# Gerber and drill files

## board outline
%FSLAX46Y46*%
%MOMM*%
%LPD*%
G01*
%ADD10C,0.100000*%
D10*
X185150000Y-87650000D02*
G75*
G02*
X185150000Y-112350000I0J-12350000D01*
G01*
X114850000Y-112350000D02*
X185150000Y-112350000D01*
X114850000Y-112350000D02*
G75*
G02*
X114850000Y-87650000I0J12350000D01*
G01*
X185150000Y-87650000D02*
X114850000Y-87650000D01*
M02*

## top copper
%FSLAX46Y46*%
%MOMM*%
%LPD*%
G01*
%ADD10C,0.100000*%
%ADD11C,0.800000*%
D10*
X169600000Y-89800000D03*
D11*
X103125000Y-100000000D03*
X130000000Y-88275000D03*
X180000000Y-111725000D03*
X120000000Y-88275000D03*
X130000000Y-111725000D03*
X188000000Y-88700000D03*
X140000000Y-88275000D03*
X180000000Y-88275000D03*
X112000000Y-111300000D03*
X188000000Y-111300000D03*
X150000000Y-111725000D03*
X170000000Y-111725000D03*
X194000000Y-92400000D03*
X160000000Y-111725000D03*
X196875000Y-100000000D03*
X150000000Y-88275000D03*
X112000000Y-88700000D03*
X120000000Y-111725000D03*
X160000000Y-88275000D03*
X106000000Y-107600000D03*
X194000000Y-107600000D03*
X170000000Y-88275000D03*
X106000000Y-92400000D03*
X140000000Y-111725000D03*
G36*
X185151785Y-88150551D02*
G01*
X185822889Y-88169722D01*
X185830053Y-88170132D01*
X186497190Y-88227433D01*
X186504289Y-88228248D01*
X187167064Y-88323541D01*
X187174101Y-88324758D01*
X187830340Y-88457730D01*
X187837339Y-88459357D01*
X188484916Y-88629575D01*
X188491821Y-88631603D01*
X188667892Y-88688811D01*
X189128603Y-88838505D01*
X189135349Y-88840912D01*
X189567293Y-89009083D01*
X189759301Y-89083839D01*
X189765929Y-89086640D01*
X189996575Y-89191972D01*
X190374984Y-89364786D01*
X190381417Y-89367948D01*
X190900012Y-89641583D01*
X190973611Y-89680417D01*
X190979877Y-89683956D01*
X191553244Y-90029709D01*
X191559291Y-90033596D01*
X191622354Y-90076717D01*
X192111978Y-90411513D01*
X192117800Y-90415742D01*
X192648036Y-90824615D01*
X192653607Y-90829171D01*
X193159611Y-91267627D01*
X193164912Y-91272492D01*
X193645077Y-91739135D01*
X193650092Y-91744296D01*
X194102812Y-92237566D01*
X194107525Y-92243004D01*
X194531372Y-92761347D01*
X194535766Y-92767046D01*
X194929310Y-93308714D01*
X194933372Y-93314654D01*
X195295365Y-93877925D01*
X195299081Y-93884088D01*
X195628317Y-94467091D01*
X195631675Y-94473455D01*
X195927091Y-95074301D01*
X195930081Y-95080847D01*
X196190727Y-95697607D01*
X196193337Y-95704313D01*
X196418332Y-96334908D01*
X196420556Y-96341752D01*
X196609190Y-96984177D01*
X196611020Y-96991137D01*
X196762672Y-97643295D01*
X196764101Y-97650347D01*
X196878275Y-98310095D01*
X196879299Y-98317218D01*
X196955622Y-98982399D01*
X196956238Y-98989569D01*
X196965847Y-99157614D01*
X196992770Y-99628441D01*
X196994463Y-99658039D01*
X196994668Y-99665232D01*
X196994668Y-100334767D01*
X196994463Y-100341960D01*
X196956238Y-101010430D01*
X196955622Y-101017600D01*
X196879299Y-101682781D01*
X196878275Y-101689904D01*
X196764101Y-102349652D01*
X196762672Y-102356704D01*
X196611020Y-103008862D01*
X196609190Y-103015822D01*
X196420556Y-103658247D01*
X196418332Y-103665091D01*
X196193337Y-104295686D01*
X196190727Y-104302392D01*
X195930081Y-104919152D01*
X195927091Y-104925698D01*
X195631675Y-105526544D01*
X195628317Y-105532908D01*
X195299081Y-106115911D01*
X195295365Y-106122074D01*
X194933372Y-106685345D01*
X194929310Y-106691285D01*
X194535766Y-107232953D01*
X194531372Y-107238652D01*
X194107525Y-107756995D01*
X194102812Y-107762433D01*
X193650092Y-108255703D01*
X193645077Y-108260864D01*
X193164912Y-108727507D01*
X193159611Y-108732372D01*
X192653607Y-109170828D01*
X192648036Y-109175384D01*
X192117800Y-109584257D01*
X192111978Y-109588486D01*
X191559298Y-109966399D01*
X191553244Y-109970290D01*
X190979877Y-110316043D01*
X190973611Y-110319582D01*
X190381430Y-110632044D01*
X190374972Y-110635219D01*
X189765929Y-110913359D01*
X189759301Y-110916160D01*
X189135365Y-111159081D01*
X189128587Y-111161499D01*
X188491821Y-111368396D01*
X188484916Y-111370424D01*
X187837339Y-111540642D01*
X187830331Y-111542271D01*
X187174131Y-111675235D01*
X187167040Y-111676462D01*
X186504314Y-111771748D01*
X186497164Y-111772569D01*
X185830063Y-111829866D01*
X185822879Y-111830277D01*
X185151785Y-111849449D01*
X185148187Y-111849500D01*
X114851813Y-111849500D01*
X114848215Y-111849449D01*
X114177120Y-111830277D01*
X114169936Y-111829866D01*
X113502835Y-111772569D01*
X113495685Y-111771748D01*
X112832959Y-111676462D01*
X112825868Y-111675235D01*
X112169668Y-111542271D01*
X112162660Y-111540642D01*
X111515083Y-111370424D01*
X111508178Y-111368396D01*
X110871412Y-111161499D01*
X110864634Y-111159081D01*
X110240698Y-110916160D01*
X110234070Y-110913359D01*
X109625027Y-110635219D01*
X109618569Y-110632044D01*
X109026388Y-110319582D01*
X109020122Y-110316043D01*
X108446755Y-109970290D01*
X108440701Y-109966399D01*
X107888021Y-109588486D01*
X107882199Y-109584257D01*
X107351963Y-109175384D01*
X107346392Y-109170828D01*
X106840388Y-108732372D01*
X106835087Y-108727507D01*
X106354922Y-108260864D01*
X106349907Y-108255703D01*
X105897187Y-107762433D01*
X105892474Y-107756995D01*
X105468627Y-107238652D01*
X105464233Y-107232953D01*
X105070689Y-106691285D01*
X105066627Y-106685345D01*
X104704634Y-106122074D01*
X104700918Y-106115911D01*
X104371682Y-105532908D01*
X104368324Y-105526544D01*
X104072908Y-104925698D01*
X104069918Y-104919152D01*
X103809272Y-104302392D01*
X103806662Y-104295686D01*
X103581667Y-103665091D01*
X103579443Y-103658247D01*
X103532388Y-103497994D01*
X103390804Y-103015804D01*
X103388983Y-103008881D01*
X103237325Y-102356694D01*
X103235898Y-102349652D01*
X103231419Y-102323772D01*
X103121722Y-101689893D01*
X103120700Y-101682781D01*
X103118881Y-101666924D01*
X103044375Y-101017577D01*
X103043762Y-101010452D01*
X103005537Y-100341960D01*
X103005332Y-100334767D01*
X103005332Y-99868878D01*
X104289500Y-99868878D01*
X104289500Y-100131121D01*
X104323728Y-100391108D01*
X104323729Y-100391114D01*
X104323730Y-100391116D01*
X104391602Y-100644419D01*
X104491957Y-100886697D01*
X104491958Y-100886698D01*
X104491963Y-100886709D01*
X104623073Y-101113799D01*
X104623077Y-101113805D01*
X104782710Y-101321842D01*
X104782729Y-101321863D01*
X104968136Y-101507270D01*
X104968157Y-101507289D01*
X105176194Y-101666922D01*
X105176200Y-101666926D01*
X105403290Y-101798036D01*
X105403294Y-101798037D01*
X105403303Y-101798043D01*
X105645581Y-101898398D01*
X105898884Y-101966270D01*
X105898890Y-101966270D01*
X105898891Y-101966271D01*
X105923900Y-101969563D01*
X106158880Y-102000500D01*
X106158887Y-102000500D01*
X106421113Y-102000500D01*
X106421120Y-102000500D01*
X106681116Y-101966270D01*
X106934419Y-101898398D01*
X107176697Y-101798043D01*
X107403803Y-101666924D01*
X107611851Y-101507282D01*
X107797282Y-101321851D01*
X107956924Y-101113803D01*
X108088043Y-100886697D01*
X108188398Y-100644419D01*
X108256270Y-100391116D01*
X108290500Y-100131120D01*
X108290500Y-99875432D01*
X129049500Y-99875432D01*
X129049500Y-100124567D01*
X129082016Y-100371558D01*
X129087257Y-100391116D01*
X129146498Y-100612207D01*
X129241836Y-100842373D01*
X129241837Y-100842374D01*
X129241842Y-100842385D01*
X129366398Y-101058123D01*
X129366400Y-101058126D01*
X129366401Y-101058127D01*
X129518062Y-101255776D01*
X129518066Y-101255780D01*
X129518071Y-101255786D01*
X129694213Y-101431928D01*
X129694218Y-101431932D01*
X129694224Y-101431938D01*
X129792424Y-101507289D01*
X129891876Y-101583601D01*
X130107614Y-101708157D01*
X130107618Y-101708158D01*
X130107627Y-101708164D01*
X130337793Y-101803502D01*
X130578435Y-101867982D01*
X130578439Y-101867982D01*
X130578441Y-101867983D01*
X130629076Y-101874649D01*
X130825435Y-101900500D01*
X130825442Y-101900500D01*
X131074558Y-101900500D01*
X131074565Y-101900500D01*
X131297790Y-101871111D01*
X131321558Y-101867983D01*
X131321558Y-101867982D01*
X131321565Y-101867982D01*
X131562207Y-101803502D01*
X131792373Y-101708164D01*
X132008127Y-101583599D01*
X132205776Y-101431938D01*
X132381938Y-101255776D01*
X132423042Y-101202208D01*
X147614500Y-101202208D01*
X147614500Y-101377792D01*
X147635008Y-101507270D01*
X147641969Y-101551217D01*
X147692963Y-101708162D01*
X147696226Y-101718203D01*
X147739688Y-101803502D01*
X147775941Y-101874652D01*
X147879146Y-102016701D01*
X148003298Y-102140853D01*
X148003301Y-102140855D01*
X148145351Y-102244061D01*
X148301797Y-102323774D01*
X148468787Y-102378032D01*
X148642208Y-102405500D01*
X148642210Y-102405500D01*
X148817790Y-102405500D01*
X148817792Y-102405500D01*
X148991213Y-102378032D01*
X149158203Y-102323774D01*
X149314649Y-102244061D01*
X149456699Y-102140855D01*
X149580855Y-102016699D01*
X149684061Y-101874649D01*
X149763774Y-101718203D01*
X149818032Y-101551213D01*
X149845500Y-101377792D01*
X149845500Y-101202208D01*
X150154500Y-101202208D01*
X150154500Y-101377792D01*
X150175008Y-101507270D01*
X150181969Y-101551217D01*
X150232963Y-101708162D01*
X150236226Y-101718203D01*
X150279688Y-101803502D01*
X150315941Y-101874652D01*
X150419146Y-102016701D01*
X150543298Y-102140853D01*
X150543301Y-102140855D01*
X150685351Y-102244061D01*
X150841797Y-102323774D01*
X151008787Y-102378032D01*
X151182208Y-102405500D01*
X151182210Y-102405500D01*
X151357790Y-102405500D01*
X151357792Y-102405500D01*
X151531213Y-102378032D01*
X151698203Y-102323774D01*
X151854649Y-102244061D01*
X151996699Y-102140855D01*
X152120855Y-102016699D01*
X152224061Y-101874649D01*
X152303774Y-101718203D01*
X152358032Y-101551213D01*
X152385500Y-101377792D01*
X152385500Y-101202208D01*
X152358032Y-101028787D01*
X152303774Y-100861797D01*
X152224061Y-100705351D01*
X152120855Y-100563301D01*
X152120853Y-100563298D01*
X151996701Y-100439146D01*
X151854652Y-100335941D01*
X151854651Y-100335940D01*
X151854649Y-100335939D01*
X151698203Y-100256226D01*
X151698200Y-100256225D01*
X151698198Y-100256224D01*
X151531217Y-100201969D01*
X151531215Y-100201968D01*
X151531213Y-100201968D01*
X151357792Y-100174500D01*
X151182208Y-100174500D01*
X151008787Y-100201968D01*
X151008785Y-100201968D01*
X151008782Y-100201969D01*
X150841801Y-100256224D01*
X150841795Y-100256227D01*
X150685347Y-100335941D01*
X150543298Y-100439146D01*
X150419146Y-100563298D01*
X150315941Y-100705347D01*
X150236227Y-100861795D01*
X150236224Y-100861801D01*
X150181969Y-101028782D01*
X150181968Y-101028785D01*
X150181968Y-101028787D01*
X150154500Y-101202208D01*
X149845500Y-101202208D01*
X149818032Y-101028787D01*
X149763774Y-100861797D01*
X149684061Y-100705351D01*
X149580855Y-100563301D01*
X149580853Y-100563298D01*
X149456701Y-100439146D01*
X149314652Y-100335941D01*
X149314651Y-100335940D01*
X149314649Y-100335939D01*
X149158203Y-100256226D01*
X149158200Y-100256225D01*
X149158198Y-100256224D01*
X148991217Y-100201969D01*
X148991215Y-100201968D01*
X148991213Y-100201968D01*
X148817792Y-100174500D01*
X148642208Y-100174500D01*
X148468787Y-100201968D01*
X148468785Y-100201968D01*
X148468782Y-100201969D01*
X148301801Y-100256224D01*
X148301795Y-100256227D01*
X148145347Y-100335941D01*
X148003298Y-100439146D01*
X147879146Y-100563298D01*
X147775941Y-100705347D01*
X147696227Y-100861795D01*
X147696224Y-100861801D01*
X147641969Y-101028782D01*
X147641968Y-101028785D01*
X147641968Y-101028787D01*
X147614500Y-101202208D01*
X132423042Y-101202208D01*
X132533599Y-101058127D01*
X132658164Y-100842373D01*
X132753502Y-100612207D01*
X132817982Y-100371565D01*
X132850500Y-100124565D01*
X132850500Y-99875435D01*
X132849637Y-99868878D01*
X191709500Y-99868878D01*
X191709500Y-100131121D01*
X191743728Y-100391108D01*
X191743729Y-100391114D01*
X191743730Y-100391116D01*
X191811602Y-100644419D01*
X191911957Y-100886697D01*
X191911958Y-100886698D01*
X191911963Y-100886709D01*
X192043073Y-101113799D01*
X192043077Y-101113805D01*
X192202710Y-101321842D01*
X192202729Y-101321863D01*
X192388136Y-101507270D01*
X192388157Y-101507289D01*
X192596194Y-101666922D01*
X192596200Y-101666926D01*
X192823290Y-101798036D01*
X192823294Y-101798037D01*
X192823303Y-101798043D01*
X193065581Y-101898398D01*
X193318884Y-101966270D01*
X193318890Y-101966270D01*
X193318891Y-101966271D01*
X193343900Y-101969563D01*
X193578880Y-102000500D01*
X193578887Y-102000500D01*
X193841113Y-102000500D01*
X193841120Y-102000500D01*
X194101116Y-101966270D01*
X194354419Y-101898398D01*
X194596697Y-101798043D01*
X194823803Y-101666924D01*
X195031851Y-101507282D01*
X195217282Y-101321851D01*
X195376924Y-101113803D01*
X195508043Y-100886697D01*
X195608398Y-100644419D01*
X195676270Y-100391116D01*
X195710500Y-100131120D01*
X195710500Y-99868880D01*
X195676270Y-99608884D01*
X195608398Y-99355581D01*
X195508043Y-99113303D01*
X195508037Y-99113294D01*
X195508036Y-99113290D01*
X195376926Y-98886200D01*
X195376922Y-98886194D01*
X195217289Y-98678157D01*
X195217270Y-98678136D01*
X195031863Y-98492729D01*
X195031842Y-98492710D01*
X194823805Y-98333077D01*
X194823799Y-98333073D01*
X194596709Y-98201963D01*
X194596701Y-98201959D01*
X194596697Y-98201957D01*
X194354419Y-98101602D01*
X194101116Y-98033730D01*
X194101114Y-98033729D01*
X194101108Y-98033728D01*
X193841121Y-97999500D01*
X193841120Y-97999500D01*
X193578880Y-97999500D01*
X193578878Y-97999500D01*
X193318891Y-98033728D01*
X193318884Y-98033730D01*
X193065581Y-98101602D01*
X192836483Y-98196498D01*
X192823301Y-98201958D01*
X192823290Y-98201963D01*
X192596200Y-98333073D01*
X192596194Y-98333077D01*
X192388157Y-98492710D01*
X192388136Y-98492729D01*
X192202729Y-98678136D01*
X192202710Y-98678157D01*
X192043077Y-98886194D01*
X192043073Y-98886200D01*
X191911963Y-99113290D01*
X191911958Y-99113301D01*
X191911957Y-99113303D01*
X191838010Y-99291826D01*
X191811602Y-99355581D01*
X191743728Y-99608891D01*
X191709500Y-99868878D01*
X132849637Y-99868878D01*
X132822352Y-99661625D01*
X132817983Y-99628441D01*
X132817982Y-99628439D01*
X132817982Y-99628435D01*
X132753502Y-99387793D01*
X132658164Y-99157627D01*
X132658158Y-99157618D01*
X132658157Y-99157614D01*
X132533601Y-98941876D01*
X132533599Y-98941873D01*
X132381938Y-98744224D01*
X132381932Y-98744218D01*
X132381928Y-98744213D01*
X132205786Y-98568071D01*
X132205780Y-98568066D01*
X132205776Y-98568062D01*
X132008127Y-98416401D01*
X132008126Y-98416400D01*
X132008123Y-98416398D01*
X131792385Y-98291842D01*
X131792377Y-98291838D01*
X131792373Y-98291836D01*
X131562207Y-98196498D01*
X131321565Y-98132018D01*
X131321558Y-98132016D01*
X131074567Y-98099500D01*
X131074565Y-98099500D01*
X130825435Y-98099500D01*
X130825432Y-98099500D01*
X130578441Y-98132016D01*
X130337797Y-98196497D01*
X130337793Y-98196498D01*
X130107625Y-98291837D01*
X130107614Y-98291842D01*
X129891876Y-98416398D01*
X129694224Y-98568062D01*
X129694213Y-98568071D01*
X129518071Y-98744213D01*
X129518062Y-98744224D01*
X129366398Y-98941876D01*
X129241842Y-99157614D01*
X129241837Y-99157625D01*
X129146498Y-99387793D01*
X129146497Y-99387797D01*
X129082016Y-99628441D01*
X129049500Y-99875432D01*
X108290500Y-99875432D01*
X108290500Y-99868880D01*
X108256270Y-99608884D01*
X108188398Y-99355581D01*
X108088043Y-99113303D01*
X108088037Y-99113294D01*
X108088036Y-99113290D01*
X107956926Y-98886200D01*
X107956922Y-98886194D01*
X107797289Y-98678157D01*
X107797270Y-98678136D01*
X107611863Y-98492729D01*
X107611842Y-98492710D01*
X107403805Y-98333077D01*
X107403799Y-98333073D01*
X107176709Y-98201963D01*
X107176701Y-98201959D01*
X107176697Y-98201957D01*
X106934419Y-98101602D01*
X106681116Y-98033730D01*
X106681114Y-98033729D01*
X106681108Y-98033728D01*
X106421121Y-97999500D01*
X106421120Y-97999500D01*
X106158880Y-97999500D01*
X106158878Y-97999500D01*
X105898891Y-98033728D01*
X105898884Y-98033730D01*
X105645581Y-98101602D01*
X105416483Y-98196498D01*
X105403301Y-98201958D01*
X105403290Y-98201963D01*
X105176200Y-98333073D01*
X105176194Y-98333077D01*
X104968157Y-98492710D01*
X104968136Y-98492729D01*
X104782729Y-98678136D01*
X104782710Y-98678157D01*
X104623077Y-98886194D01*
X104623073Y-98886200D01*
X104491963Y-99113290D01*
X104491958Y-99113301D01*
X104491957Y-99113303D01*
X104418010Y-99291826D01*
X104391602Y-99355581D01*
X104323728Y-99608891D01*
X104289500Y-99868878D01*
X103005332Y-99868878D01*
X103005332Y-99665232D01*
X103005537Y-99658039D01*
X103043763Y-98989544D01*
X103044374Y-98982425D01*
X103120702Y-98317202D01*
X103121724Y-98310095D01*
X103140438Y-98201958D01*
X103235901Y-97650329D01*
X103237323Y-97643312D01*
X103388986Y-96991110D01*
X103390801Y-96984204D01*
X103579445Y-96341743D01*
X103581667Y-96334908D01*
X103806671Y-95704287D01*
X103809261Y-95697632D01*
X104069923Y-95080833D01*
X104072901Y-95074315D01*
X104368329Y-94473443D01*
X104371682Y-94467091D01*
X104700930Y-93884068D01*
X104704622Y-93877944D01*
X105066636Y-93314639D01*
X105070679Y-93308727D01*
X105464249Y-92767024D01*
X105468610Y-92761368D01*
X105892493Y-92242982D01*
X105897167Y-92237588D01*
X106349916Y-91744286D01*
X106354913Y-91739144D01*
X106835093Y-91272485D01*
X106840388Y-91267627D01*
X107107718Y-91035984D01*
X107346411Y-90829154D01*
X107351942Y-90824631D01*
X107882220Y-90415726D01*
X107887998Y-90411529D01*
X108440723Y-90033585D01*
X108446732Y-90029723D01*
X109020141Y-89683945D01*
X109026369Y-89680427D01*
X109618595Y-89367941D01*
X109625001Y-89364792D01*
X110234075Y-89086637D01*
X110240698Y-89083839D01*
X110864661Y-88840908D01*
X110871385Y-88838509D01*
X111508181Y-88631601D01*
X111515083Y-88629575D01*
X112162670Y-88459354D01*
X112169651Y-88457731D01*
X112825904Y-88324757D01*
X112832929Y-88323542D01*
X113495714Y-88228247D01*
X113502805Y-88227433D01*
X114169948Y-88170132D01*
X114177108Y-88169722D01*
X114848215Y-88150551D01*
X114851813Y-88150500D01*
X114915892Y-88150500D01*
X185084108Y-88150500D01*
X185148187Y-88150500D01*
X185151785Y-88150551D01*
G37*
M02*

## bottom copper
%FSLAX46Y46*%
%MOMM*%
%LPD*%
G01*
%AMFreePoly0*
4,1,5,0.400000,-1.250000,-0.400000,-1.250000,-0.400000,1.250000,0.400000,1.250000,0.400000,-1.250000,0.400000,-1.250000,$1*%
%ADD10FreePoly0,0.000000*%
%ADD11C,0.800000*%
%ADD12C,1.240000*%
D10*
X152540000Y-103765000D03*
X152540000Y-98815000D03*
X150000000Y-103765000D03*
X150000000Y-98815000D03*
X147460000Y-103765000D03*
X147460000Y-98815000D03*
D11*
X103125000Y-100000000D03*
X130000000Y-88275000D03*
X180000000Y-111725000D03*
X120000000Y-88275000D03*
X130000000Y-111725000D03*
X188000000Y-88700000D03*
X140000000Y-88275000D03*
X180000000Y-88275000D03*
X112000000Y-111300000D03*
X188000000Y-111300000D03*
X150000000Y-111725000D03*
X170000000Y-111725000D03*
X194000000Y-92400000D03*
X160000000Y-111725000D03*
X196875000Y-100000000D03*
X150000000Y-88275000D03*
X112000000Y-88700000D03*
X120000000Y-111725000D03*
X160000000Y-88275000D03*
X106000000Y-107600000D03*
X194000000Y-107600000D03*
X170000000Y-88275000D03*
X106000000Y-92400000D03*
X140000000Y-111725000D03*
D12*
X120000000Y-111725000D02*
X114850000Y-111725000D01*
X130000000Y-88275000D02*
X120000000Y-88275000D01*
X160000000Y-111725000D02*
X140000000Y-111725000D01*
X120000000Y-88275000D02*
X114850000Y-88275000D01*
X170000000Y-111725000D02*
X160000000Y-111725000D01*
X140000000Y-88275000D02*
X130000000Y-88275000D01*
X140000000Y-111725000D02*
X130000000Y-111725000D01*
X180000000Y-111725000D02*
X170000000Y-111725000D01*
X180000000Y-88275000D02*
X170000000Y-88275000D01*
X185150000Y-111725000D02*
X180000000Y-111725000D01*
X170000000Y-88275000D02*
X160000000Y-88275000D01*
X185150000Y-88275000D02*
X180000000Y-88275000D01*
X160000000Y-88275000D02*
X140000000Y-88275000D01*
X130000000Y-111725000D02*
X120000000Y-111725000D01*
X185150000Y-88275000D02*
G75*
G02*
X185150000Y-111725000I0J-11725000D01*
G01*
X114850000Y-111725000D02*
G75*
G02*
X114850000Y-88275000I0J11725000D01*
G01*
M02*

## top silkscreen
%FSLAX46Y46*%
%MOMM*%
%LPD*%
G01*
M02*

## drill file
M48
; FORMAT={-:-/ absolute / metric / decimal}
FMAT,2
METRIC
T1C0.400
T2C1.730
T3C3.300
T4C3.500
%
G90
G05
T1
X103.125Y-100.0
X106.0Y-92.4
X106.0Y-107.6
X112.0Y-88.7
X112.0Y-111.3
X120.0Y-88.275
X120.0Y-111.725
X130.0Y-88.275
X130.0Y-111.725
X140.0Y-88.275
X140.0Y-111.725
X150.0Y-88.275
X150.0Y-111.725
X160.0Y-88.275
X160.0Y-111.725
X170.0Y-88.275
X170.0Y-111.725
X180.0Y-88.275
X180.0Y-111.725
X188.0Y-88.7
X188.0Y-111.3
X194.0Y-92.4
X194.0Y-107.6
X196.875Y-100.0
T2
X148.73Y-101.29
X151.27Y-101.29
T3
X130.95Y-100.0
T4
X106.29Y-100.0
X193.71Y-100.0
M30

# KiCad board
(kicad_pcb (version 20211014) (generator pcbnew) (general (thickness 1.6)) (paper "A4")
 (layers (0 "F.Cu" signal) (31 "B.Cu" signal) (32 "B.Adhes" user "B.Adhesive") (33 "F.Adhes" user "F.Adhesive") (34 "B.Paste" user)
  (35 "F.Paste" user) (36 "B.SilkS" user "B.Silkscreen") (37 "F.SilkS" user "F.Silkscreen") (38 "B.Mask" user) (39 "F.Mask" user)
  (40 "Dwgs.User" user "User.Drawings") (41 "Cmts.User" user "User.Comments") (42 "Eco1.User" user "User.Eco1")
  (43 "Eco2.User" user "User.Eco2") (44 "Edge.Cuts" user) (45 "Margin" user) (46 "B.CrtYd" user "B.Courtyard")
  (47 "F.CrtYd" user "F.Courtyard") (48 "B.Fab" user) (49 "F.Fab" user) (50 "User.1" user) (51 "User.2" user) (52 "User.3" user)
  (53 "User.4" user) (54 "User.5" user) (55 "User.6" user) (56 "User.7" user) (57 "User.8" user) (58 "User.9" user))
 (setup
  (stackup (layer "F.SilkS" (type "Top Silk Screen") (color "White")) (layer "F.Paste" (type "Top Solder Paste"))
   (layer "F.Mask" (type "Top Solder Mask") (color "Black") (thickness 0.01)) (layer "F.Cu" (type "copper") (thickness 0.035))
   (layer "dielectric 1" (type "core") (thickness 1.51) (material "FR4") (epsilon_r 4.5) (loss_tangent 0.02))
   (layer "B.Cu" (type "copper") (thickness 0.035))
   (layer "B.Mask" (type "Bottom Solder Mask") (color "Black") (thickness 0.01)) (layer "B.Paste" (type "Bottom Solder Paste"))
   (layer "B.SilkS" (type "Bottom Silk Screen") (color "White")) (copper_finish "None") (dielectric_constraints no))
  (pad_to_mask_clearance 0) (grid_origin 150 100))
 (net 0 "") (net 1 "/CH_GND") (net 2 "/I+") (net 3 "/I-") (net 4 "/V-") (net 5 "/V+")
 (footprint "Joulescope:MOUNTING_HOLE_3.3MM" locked (layer "F.Cu") (at 130.95 100)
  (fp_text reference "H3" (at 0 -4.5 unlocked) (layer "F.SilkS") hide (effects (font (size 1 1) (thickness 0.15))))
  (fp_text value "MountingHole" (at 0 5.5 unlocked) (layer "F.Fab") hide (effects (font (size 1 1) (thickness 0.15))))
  (pad "" np_thru_hole circle locked (at 0 0) (size 3.3 3.3) (drill 3.3) (layers *.Mask)))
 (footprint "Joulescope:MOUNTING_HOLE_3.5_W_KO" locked (layer "F.Cu") (at 193.71 100)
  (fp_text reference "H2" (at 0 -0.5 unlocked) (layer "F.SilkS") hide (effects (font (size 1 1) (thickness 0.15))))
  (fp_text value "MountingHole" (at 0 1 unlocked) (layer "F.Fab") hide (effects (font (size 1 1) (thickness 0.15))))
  (pad "" np_thru_hole circle locked (at 0 0) (size 3.5 3.5) (drill 3.5) (layers *.Mask))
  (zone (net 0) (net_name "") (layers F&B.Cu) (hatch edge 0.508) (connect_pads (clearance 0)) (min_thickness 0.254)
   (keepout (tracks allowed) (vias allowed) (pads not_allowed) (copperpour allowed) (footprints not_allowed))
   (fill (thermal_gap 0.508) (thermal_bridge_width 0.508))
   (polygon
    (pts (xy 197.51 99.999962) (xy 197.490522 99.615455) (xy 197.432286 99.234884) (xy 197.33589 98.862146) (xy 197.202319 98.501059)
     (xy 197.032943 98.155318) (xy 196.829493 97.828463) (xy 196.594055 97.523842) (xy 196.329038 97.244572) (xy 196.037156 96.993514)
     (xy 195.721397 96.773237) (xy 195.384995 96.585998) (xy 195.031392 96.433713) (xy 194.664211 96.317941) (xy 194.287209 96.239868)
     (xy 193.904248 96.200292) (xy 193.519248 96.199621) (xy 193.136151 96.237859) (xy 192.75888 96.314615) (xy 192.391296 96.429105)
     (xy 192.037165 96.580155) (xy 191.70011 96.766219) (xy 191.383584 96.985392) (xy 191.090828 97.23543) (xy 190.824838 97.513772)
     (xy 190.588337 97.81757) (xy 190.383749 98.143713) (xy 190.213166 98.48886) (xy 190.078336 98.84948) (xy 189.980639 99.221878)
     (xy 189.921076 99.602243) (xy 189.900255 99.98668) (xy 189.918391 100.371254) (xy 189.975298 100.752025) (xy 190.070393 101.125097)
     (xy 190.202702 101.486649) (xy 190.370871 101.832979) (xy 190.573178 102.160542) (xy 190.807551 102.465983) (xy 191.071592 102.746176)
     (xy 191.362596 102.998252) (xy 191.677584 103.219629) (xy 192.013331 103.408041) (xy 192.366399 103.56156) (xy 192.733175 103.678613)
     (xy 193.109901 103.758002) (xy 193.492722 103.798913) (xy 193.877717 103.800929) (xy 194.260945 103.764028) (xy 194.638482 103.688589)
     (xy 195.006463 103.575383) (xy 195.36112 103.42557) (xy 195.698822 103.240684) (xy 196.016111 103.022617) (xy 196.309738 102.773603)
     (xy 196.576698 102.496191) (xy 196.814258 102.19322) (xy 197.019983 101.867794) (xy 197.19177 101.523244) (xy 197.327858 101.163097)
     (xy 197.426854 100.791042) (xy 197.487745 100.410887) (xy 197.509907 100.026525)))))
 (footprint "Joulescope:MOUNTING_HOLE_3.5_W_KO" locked (layer "F.Cu") (at 106.29 100)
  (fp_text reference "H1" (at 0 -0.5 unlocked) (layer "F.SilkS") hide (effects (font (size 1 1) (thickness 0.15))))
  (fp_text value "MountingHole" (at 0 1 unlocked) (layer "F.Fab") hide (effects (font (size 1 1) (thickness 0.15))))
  (pad "" np_thru_hole circle locked (at 0 0) (size 3.5 3.5) (drill 3.5) (layers *.Mask))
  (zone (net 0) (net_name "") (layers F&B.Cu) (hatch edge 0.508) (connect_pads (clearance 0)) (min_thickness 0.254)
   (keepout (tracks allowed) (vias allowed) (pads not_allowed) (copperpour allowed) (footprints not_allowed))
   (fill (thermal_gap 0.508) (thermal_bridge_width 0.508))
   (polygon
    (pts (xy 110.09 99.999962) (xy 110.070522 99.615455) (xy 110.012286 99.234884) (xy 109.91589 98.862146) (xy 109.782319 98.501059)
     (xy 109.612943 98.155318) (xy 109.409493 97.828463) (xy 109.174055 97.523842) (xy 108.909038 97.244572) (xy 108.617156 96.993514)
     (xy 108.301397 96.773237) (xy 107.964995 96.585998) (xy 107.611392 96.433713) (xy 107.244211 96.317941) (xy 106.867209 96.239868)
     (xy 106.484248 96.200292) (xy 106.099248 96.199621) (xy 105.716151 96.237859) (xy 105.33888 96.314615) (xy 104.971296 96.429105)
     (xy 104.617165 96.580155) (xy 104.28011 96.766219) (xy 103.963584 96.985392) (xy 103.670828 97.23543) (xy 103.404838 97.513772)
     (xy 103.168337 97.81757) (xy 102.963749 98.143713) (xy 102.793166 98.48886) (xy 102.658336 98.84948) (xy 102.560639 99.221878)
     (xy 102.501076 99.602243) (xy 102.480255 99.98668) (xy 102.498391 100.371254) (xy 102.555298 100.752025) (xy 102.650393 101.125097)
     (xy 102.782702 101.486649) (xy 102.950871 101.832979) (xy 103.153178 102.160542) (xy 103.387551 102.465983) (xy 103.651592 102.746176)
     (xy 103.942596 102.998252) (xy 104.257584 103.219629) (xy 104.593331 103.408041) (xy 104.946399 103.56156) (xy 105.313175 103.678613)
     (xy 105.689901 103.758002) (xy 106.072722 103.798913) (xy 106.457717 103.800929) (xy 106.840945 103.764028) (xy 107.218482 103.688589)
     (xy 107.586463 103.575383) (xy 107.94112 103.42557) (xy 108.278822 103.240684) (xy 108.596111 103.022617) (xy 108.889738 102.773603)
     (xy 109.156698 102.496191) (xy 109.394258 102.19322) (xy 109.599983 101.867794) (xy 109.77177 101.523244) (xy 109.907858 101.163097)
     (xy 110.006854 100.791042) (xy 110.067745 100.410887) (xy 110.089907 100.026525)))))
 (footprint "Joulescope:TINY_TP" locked (layer "F.Cu") (at 169.6 89.5)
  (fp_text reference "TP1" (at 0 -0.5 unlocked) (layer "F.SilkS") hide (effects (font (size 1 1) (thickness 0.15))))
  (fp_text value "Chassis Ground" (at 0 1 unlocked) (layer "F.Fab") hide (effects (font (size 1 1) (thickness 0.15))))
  (pad "1" smd circle locked (at 0 0.3) (size 0.1 0.1) (layers "F.Cu" "F.Paste" "F.Mask") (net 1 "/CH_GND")))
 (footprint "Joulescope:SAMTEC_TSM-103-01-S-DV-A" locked (layer "B.Cu") (at 150 101.29)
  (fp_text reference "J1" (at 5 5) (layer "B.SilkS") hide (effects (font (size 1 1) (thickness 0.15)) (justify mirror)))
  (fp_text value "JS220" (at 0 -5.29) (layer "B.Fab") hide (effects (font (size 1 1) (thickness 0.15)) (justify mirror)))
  (pad "" np_thru_hole circle locked (at 1.27 0) (size 1.73 1.73) (drill 1.73) (layers *.Cu *.Mask))
  (pad "" np_thru_hole circle locked (at -1.27 0) (size 1.73 1.73) (drill 1.73) (layers *.Cu *.Mask))
  (pad "1" smd custom locked (at 2.54 2.475) (size 0.8 2.5) (layers "B.Cu") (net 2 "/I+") (zone_connect 0)
   (options (clearance outline) (anchor rect)) (primitives))
  (pad "2" smd custom locked (at 2.54 -2.475) (size 0.8 2.5) (layers "B.Cu") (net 2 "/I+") (zone_connect 0)
   (options (clearance outline) (anchor rect)) (primitives))
  (pad "3" smd custom locked (at 0 2.475) (size 0.8 2.5) (layers "B.Cu") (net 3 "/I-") (zone_connect 0)
   (options (clearance outline) (anchor rect)) (primitives))
  (pad "4" smd custom locked (at 0 -2.475) (size 0.8 2.5) (layers "B.Cu") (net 3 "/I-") (zone_connect 0)
   (options (clearance outline) (anchor rect)) (primitives))
  (pad "5" smd custom locked (at -2.54 2.475) (size 0.8 2.5) (layers "B.Cu") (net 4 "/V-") (zone_connect 0)
   (options (clearance outline) (anchor rect)) (primitives))
  (pad "6" smd custom locked (at -2.54 -2.475) (size 0.8 2.5) (layers "B.Cu") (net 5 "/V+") (zone_connect 0)
   (options (clearance outline) (anchor rect)) (primitives)))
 (gr_arc locked (start 185.15 87.65) (mid 197.5 100) (end 185.15 112.35) (layer "Edge.Cuts") (width 0.1))
 (gr_line locked (start 114.85 112.35) (end 185.15 112.35) (layer "Edge.Cuts") (width 0.1))
 (gr_arc locked (start 114.85 112.35) (mid 102.5 100) (end 114.85 87.65) (layer "Edge.Cuts") (width 0.1))
 (gr_line locked (start 185.15 87.65) (end 114.85 87.65) (layer "Edge.Cuts") (width 0.1))
 (via locked (at 103.125 100) (size 0.8) (drill 0.4) (layers "F.Cu" "B.Cu") (free) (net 1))
 (via locked (at 130 88.275) (size 0.8) (drill 0.4) (layers "F.Cu" "B.Cu") (free) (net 1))
 (via locked (at 180 111.725) (size 0.8) (drill 0.4) (layers "F.Cu" "B.Cu") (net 1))
 (via locked (at 120 88.275) (size 0.8) (drill 0.4) (layers "F.Cu" "B.Cu") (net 1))
 (via locked (at 130 111.725) (size 0.8) (drill 0.4) (layers "F.Cu" "B.Cu") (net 1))
 (via locked (at 188 88.7) (size 0.8) (drill 0.4) (layers "F.Cu" "B.Cu") (free) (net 1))
 (via locked (at 140 88.275) (size 0.8) (drill 0.4) (layers "F.Cu" "B.Cu") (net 1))
 (via locked (at 180 88.275) (size 0.8) (drill 0.4) (layers "F.Cu" "B.Cu") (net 1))
 (via locked (at 112 111.3) (size 0.8) (drill 0.4) (layers "F.Cu" "B.Cu") (free) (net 1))
 (via locked (at 188 111.3) (size 0.8) (drill 0.4) (layers "F.Cu" "B.Cu") (free) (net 1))
 (via locked (at 150 111.725) (size 0.8) (drill 0.4) (layers "F.Cu" "B.Cu") (free) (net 1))
 (via locked (at 170 111.725) (size 0.8) (drill 0.4) (layers "F.Cu" "B.Cu") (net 1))
 (via locked (at 194 92.4) (size 0.8) (drill 0.4) (layers "F.Cu" "B.Cu") (free) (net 1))
 (via locked (at 160 111.725) (size 0.8) (drill 0.4) (layers "F.Cu" "B.Cu") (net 1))
 (via locked (at 196.875 100) (size 0.8) (drill 0.4) (layers "F.Cu" "B.Cu") (free) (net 1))
 (via locked (at 150 88.275) (size 0.8) (drill 0.4) (layers "F.Cu" "B.Cu") (free) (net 1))
 (via locked (at 112 88.7) (size 0.8) (drill 0.4) (layers "F.Cu" "B.Cu") (free) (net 1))
 (via locked (at 120 111.725) (size 0.8) (drill 0.4) (layers "F.Cu" "B.Cu") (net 1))
 (via locked (at 160 88.275) (size 0.8) (drill 0.4) (layers "F.Cu" "B.Cu") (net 1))
 (via locked (at 106 107.6) (size 0.8) (drill 0.4) (layers "F.Cu" "B.Cu") (free) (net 1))
 (via locked (at 194 107.6) (size 0.8) (drill 0.4) (layers "F.Cu" "B.Cu") (free) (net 1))
 (via locked (at 170 88.275) (size 0.8) (drill 0.4) (layers "F.Cu" "B.Cu") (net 1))
 (via locked (at 106 92.4) (size 0.8) (drill 0.4) (layers "F.Cu" "B.Cu") (free) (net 1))
 (via locked (at 140 111.725) (size 0.8) (drill 0.4) (layers "F.Cu" "B.Cu") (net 1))
 (segment locked (start 120 111.725) (end 114.85 111.725) (width 1.24) (layer "B.Cu") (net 1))
 (segment locked (start 130 88.275) (end 120 88.275) (width 1.24) (layer "B.Cu") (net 1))
 (segment locked (start 160 111.725) (end 140 111.725) (width 1.24) (layer "B.Cu") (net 1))
 (segment locked (start 120 88.275) (end 114.85 88.275) (width 1.24) (layer "B.Cu") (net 1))
 (segment locked (start 170 111.725) (end 160 111.725) (width 1.24) (layer "B.Cu") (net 1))
 (segment locked (start 140 88.275) (end 130 88.275) (width 1.24) (layer "B.Cu") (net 1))
 (segment locked (start 140 111.725) (end 130 111.725) (width 1.24) (layer "B.Cu") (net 1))
 (segment locked (start 180 111.725) (end 170 111.725) (width 1.24) (layer "B.Cu") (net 1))
 (segment locked (start 180 88.275) (end 170 88.275) (width 1.24) (layer "B.Cu") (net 1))
 (segment locked (start 185.15 111.725) (end 180 111.725) (width 1.24) (layer "B.Cu") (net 1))
 (segment locked (start 170 88.275) (end 160 88.275) (width 1.24) (layer "B.Cu") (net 1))
 (segment locked (start 185.15 88.275) (end 180 88.275) (width 1.24) (layer "B.Cu") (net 1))
 (segment locked (start 160 88.275) (end 140 88.275) (width 1.24) (layer "B.Cu") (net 1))
 (segment locked (start 130 111.725) (end 120 111.725) (width 1.24) (layer "B.Cu") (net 1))
 (arc locked (start 185.15 88.275) (mid 196.875 100) (end 185.15 111.725) (width 1.24) (layer "B.Cu") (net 1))
 (arc locked (start 114.85 111.725) (mid 103.125 100) (end 114.85 88.275) (width 1.24) (layer "B.Cu") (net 1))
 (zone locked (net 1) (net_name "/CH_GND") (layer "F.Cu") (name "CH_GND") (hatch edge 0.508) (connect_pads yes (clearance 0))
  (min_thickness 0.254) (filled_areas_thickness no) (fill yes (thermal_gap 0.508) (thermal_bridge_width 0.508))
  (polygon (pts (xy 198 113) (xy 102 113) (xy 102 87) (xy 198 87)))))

